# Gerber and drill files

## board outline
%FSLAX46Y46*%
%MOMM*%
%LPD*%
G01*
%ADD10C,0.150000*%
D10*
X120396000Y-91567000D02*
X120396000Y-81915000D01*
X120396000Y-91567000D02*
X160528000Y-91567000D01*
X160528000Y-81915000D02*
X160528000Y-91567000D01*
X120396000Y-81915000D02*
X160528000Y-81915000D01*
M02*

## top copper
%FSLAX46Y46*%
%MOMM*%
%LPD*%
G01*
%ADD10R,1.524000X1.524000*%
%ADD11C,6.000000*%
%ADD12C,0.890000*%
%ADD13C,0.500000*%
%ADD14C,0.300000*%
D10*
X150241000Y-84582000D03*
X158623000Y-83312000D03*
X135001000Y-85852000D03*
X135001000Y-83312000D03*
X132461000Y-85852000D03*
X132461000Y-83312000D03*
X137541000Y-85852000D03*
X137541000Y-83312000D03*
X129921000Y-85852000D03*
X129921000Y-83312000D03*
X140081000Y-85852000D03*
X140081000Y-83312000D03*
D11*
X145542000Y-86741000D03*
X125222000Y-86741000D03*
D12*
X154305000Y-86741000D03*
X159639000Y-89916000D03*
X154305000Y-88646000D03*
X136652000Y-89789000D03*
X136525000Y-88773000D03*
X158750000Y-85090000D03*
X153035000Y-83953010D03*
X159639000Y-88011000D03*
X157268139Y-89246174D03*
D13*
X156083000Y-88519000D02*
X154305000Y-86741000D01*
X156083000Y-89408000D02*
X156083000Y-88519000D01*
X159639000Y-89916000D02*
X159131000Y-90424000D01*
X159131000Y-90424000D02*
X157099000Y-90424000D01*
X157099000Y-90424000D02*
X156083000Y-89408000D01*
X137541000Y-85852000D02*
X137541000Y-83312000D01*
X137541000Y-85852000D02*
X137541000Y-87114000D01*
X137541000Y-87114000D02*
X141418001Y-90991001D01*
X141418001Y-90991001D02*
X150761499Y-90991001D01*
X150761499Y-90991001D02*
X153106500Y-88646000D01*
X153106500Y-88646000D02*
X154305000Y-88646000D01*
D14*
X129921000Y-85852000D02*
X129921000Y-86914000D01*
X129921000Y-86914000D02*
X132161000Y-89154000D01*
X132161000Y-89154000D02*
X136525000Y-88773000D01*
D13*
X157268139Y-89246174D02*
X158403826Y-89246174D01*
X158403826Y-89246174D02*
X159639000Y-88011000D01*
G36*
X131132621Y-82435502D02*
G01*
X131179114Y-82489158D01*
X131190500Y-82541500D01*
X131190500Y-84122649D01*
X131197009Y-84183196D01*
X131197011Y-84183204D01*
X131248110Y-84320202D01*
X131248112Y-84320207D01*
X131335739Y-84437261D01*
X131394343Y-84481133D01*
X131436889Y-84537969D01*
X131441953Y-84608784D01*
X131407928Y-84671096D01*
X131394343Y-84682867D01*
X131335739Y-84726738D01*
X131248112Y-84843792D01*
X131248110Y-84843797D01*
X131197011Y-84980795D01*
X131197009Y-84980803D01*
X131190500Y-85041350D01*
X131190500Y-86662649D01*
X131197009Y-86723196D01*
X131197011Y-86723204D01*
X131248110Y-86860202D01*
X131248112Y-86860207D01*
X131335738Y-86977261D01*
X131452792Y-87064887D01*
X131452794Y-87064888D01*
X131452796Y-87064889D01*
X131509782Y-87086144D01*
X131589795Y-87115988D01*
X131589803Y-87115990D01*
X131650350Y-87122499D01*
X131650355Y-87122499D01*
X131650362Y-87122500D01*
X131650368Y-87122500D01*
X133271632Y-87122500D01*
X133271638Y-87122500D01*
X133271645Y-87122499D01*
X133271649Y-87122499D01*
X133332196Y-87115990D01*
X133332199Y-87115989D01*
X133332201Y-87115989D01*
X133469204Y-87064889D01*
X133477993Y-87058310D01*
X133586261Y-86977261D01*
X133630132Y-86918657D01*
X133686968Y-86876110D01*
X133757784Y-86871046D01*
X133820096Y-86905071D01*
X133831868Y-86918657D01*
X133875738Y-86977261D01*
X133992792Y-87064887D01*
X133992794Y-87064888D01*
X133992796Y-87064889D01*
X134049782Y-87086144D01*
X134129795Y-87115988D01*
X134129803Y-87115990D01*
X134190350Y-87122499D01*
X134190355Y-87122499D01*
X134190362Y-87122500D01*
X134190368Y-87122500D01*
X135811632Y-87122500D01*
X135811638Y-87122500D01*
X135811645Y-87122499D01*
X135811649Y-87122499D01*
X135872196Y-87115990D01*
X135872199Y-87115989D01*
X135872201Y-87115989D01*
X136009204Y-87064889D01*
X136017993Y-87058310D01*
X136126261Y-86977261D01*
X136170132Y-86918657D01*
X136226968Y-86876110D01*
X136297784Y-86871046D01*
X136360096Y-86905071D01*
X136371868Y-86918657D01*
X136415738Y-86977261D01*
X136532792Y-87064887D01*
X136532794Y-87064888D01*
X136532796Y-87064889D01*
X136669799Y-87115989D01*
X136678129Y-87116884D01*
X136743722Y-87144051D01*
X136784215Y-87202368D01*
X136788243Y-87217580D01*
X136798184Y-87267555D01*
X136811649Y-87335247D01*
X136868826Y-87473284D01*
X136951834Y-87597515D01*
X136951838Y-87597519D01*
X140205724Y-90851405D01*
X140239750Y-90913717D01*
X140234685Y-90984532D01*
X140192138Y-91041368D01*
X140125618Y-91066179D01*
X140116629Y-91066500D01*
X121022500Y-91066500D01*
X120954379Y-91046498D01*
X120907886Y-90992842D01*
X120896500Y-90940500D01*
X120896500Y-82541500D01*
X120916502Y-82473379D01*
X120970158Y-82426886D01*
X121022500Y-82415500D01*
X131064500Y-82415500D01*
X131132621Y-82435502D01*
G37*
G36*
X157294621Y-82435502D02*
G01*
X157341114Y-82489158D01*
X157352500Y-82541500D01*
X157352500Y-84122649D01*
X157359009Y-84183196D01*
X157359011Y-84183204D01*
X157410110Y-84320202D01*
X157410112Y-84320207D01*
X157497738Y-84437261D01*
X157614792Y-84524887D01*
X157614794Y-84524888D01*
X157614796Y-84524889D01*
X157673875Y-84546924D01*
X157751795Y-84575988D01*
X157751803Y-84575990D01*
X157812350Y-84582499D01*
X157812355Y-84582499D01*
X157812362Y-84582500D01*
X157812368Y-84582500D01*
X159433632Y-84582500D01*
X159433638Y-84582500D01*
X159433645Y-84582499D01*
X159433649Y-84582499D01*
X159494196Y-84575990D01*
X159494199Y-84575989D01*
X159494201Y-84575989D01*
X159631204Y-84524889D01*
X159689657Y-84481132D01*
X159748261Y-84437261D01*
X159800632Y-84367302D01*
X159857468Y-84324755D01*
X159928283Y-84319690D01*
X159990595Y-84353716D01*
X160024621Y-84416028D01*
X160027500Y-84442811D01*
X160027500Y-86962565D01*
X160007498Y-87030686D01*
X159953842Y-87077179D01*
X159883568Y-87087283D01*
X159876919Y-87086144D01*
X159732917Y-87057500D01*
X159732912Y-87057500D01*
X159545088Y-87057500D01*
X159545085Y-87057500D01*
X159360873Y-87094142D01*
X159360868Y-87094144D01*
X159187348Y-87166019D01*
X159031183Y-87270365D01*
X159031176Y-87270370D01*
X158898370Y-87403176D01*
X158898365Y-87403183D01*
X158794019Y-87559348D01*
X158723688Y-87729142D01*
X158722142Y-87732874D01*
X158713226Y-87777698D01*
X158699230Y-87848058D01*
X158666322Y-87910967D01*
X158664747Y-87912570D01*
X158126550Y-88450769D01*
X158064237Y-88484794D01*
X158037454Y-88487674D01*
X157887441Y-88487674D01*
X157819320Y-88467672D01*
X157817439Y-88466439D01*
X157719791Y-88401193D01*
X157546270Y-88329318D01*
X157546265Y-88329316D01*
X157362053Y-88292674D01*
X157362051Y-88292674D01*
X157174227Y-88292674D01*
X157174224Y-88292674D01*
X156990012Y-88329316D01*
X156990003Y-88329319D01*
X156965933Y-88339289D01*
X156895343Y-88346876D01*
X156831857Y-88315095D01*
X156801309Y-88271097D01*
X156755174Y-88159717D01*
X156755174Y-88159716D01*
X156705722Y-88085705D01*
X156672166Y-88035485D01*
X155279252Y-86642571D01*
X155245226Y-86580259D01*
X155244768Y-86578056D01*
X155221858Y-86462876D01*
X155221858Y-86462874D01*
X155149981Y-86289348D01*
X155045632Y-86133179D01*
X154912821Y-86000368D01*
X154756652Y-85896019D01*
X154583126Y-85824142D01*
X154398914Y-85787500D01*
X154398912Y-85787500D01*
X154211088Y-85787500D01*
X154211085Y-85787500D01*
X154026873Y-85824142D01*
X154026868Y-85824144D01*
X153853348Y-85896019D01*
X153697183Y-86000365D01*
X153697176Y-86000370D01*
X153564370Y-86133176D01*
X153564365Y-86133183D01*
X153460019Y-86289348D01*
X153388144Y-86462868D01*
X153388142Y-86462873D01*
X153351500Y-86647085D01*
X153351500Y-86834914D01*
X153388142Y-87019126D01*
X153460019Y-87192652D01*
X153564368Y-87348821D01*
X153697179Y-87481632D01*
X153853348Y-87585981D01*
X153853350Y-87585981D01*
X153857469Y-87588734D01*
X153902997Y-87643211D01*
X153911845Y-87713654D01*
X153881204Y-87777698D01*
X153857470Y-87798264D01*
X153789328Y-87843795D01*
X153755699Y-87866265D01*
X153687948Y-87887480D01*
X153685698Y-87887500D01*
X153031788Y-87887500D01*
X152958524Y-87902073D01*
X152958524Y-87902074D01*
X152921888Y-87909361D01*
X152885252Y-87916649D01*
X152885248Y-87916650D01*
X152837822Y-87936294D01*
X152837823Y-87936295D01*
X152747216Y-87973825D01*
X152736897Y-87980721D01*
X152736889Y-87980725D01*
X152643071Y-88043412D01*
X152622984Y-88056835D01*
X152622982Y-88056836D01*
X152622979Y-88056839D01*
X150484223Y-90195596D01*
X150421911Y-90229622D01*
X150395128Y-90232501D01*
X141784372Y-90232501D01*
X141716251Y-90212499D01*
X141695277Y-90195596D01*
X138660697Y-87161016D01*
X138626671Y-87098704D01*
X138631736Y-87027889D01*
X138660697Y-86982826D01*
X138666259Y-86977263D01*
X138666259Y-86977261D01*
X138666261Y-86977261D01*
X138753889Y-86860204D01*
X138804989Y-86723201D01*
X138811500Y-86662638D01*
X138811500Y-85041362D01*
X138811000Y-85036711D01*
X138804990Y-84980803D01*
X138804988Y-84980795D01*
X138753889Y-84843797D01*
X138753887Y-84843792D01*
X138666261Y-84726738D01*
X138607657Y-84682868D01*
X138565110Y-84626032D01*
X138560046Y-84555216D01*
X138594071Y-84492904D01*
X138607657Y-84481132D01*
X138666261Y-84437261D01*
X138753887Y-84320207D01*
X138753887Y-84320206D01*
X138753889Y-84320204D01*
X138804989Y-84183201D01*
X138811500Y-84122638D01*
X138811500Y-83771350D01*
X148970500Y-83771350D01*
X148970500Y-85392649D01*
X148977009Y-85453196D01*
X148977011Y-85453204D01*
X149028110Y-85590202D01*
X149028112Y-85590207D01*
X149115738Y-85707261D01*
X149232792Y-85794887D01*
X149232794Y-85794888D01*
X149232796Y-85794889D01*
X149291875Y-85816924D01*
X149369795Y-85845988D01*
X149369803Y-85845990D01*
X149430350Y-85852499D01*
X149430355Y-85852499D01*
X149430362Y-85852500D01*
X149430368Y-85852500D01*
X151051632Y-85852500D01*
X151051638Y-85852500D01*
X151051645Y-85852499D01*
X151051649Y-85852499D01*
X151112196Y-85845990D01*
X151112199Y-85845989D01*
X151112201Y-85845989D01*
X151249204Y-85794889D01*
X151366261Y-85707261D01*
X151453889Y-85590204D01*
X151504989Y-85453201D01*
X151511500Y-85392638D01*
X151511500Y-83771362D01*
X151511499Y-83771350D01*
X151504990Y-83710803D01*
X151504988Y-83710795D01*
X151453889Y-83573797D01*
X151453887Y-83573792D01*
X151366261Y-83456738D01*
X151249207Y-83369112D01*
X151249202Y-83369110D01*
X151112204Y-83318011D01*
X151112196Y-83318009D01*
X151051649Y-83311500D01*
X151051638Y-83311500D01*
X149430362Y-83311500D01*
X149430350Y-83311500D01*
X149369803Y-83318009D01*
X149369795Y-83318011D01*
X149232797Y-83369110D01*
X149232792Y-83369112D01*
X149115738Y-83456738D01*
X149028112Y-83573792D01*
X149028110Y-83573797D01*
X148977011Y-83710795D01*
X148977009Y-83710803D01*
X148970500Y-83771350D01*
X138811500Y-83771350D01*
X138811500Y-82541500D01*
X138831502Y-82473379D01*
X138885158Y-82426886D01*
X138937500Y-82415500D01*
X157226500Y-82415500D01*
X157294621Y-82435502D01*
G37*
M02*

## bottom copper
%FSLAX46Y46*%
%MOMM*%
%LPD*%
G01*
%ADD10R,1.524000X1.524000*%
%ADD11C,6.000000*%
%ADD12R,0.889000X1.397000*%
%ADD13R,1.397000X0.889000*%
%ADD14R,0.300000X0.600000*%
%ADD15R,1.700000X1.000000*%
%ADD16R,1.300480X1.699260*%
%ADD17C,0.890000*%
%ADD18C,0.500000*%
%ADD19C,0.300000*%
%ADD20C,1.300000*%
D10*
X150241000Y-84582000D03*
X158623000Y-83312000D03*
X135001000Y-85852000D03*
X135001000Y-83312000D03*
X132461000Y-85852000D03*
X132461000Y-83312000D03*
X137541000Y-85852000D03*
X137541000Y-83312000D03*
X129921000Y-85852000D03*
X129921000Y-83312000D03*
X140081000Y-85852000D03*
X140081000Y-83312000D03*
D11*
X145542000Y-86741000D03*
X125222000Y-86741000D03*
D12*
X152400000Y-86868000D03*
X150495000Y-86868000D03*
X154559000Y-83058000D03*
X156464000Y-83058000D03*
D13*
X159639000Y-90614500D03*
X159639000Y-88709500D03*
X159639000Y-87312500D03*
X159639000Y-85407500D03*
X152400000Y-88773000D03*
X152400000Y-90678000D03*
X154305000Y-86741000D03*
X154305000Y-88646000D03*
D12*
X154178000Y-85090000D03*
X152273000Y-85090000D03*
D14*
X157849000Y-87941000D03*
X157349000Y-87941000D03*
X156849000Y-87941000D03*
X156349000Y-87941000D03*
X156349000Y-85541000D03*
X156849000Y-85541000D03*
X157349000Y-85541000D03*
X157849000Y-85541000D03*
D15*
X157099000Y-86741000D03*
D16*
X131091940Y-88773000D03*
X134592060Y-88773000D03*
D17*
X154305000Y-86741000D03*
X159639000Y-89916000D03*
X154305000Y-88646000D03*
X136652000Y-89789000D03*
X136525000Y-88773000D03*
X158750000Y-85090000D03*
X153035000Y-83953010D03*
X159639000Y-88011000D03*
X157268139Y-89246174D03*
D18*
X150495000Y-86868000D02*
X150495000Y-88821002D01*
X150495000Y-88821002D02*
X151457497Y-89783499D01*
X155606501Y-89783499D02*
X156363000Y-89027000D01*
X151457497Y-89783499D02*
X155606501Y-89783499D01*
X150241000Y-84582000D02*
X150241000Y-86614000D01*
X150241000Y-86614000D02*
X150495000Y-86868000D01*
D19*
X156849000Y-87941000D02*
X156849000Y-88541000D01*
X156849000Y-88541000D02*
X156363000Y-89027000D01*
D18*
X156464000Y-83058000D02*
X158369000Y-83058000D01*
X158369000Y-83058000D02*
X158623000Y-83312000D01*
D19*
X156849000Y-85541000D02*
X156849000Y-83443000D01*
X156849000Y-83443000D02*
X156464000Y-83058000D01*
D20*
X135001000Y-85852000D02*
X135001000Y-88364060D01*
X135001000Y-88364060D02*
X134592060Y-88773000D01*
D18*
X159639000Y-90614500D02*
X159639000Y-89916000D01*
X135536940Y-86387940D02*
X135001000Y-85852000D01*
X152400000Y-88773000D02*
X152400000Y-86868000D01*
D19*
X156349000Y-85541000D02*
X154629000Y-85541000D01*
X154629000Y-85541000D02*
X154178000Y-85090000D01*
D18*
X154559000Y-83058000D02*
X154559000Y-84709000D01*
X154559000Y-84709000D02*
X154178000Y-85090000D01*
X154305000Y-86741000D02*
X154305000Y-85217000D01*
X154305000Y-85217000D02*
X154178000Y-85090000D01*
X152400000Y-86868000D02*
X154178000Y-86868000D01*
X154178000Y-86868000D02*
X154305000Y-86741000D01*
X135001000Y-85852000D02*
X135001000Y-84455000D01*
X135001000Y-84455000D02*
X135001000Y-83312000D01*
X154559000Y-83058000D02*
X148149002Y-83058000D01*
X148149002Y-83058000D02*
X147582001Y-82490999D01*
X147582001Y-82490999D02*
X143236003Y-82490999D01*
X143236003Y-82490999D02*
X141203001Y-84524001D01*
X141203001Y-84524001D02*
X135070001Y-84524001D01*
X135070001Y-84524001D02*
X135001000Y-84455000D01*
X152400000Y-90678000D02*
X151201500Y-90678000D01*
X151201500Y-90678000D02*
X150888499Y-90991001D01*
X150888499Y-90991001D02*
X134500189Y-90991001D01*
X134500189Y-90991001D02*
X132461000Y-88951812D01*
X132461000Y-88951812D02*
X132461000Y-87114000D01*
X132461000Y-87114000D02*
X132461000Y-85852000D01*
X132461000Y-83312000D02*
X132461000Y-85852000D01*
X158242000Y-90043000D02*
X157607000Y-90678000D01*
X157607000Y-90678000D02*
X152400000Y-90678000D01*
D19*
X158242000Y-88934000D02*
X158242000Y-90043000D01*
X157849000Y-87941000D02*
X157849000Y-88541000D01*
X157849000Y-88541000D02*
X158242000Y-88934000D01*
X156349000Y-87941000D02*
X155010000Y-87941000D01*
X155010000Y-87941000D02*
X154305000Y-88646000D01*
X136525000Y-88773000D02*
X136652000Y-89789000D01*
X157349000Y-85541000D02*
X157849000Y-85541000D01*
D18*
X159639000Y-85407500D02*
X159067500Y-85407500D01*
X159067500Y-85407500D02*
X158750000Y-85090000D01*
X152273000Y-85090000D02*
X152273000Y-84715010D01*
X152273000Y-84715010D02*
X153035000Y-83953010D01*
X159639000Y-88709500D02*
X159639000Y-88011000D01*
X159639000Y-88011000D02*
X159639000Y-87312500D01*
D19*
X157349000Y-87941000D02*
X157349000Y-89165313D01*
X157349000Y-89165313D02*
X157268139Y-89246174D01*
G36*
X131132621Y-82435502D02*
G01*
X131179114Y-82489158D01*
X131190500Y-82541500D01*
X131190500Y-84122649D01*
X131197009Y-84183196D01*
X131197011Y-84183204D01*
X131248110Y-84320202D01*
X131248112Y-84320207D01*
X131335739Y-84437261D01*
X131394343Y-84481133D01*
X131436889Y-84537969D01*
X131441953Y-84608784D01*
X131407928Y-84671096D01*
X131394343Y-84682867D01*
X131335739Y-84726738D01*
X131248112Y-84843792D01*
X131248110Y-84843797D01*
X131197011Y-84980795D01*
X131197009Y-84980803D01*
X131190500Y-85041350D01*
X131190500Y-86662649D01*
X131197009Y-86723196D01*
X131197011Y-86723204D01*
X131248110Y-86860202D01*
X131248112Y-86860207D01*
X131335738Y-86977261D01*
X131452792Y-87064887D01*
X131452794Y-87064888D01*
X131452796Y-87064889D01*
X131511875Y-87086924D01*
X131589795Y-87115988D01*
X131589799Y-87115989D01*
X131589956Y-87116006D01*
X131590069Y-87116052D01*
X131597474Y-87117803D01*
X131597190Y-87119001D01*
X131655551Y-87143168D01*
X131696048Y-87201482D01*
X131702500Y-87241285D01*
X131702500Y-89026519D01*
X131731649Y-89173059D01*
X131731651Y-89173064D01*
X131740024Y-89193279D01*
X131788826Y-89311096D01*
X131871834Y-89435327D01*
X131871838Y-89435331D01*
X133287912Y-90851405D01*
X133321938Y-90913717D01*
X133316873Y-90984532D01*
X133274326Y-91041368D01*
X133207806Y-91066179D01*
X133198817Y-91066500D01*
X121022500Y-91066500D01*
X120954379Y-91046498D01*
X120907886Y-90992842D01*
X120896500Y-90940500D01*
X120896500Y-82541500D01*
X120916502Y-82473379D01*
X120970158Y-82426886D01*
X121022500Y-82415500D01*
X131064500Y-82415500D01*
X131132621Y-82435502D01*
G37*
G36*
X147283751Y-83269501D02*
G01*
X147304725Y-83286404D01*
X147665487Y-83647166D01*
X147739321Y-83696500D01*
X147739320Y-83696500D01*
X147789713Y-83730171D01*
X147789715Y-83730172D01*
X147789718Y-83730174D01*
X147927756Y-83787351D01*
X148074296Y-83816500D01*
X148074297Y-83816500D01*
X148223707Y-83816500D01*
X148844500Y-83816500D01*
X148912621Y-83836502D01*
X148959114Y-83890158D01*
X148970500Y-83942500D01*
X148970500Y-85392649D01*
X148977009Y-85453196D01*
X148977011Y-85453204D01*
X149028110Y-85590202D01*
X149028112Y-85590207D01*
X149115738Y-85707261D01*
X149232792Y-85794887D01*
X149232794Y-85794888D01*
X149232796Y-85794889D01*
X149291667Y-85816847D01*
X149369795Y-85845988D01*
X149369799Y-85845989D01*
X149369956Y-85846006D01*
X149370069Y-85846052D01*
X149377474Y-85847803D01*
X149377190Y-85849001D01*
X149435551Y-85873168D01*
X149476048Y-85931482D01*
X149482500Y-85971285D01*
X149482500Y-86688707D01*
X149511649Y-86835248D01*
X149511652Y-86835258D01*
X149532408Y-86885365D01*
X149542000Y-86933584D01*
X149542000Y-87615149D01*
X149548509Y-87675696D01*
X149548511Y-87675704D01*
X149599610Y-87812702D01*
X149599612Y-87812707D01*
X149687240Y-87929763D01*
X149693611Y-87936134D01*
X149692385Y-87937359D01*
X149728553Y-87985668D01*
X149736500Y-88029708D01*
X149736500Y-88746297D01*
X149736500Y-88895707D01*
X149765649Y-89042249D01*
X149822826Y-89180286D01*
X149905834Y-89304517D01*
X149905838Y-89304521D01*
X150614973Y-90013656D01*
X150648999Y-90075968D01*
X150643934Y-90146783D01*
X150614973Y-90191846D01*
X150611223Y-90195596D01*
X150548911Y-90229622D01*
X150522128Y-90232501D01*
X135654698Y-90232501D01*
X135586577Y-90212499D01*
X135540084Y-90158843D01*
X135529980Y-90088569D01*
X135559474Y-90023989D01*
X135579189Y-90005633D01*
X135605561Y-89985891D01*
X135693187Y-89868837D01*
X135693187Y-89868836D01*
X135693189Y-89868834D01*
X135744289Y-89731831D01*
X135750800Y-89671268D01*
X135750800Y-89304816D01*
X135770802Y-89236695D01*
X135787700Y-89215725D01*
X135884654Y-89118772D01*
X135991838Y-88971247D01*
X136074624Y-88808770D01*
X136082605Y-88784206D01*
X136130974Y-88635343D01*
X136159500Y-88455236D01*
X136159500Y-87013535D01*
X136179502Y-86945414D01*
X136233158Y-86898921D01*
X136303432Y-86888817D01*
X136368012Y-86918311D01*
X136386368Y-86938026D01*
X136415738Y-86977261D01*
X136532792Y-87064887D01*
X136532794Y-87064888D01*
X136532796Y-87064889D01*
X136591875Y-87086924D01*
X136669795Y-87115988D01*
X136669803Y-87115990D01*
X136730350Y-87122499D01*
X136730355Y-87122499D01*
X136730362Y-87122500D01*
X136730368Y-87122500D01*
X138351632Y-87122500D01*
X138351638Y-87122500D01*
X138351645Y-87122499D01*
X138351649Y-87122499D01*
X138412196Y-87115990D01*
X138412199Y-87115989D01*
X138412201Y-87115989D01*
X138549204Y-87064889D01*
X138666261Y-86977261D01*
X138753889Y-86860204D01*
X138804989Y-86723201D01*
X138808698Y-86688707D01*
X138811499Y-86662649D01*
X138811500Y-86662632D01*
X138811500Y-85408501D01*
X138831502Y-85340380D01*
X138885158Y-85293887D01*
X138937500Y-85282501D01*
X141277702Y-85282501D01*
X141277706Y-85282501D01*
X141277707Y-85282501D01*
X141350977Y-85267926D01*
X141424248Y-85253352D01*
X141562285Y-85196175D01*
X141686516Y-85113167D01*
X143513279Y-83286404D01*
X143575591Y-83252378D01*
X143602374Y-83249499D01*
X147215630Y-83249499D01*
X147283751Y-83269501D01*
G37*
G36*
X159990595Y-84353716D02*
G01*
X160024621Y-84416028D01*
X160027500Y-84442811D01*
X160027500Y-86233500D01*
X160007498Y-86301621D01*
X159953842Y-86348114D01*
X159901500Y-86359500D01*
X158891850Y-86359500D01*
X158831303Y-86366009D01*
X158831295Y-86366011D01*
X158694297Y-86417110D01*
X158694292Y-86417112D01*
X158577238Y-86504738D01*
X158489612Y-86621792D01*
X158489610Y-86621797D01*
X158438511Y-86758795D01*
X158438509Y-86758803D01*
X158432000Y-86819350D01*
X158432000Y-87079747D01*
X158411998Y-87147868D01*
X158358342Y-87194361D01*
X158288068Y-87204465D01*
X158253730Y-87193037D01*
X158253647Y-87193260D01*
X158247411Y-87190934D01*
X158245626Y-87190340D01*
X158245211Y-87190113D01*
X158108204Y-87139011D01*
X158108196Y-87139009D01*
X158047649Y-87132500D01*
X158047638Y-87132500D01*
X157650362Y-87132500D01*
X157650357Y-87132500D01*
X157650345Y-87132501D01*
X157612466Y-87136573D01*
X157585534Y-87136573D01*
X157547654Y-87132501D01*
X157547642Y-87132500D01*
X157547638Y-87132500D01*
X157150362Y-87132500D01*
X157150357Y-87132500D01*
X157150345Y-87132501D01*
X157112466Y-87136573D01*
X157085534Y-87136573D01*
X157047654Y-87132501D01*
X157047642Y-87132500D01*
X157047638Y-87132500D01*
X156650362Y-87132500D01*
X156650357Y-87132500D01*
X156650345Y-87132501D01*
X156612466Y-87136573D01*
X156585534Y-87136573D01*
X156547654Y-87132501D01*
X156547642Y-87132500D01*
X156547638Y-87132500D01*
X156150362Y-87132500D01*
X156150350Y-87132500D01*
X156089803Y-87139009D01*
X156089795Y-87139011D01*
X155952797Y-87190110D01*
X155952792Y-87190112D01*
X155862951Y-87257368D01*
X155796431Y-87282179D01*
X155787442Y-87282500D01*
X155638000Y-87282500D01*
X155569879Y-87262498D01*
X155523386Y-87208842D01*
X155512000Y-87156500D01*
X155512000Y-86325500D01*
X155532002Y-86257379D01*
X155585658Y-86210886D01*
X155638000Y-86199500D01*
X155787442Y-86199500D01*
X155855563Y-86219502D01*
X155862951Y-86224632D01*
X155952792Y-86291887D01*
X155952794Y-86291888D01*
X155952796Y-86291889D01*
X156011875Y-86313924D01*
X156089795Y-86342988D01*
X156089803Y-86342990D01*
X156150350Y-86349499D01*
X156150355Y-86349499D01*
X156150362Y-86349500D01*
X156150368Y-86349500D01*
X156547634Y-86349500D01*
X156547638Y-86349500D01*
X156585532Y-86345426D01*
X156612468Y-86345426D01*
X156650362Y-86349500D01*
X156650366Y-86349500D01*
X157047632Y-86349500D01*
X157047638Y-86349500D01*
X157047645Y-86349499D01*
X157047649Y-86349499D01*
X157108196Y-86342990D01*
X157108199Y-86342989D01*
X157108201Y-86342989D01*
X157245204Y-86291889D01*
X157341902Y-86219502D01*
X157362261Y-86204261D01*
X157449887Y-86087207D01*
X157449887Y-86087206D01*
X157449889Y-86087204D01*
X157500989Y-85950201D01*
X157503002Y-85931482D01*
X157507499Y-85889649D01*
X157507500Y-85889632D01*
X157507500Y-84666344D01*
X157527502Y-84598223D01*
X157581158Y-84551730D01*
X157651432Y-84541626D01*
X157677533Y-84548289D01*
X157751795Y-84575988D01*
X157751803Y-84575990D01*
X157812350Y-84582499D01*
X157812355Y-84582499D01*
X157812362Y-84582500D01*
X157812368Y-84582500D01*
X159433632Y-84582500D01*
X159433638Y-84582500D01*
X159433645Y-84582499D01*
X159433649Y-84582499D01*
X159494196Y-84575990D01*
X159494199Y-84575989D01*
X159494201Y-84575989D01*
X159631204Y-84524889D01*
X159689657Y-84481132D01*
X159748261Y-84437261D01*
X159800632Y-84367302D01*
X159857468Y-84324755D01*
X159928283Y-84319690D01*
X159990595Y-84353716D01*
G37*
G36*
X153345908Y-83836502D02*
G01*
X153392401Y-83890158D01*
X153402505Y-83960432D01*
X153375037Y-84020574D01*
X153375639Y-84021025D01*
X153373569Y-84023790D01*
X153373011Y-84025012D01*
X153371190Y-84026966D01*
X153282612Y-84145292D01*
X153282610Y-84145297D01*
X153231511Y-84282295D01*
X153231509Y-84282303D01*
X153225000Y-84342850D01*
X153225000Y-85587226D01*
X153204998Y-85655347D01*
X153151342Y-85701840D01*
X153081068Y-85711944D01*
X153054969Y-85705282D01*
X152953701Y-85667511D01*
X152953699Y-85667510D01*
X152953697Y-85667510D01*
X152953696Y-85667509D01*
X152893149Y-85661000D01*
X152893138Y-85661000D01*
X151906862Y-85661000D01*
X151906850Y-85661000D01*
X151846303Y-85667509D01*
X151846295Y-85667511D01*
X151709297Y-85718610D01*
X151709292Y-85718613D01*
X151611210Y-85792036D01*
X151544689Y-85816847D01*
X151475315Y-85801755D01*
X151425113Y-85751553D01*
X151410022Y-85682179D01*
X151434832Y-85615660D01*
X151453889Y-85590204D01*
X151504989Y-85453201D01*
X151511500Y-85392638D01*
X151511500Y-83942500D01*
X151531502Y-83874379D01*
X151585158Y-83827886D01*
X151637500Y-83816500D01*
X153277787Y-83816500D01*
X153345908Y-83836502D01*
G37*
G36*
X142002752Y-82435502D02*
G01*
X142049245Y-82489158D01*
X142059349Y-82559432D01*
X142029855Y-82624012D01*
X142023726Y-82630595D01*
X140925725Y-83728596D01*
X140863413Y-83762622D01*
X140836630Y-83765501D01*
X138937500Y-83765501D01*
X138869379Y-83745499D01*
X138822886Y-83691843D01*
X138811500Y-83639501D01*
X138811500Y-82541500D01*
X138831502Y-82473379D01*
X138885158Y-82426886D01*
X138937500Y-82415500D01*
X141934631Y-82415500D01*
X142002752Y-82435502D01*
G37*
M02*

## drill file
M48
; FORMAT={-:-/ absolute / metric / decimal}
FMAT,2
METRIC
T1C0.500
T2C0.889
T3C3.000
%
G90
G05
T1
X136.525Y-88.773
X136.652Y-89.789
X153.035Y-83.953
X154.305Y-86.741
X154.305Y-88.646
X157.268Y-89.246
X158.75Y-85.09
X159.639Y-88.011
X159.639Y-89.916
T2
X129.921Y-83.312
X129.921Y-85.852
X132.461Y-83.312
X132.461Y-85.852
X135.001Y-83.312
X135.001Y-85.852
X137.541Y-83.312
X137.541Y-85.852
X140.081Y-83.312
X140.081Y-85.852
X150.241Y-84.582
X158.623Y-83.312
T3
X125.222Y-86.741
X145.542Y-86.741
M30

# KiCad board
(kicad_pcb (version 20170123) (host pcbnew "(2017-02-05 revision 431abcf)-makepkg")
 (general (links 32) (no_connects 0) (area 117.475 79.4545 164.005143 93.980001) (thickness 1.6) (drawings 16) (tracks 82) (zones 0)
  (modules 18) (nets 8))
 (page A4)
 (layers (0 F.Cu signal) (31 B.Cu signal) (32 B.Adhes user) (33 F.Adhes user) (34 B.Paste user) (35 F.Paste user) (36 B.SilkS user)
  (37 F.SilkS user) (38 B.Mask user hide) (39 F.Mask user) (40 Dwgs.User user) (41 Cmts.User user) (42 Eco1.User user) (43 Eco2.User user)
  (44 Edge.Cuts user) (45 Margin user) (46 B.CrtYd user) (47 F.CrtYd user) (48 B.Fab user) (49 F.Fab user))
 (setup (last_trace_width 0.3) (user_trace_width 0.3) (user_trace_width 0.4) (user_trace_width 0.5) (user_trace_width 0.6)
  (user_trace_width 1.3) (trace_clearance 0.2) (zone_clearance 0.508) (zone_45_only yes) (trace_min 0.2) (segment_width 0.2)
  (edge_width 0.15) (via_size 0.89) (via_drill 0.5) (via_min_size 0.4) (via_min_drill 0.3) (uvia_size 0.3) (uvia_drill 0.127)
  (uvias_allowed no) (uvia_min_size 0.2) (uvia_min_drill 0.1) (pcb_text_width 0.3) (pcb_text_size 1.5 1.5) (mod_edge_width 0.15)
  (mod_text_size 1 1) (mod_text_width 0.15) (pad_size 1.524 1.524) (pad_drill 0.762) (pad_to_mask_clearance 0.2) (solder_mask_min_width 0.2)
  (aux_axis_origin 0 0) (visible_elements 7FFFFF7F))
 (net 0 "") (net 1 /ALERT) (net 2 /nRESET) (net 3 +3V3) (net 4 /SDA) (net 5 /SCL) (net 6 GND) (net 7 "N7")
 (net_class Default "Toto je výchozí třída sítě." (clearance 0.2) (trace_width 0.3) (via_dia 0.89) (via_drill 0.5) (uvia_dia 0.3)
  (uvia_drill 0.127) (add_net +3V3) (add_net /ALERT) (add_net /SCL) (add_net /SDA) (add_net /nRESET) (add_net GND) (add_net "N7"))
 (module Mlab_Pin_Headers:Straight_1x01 (layer F.Cu) (at 150.241 84.582)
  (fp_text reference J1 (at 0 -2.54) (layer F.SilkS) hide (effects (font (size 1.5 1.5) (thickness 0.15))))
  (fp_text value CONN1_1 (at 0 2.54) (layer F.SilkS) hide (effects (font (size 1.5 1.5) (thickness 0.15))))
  (pad 1 thru_hole rect (at 0 0) (size 1.524 1.524) (drill 0.889) (layers *.Cu *.Mask F.SilkS) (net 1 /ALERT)))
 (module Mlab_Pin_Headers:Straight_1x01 (layer F.Cu) (at 158.623 83.312)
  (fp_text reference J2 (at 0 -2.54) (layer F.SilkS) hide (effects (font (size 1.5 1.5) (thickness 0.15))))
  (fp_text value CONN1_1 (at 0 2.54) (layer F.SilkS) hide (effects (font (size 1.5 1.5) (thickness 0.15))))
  (pad 1 thru_hole rect (at 0 0) (size 1.524 1.524) (drill 0.889) (layers *.Cu *.Mask F.SilkS) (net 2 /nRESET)))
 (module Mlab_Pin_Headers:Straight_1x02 (layer F.Cu) (at 135.001 84.582)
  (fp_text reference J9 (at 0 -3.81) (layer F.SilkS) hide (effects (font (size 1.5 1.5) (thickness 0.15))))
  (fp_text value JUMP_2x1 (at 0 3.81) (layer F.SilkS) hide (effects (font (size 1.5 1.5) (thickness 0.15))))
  (pad 2 thru_hole rect (at 0 1.27) (size 1.524 1.524) (drill 0.889) (layers *.Cu *.Mask F.SilkS) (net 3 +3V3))
  (pad 1 thru_hole rect (at 0 -1.27) (size 1.524 1.524) (drill 0.889) (layers *.Cu *.Mask F.SilkS) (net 3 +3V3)))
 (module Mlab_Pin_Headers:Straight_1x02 (layer F.Cu) (at 132.461 84.582)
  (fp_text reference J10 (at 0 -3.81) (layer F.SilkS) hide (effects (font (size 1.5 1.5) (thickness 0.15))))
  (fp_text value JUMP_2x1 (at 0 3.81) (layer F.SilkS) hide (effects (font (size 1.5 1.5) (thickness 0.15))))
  (pad 2 thru_hole rect (at 0 1.27) (size 1.524 1.524) (drill 0.889) (layers *.Cu *.Mask F.SilkS) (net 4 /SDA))
  (pad 1 thru_hole rect (at 0 -1.27) (size 1.524 1.524) (drill 0.889) (layers *.Cu *.Mask F.SilkS) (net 4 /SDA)))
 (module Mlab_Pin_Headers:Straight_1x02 (layer F.Cu) (at 137.541 84.582)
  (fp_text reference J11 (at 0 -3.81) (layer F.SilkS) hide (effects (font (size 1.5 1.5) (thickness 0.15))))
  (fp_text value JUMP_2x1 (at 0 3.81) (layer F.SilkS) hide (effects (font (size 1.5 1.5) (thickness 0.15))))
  (pad 2 thru_hole rect (at 0 1.27) (size 1.524 1.524) (drill 0.889) (layers *.Cu *.Mask F.SilkS) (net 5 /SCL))
  (pad 1 thru_hole rect (at 0 -1.27) (size 1.524 1.524) (drill 0.889) (layers *.Cu *.Mask F.SilkS) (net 5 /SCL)))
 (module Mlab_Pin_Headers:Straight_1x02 (layer F.Cu) (at 129.921 84.582)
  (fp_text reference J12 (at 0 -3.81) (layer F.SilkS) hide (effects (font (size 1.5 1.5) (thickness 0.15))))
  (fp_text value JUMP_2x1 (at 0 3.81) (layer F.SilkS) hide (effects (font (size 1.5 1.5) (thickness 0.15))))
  (pad 2 thru_hole rect (at 0 1.27) (size 1.524 1.524) (drill 0.889) (layers *.Cu *.Mask F.SilkS) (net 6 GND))
  (pad 1 thru_hole rect (at 0 -1.27) (size 1.524 1.524) (drill 0.889) (layers *.Cu *.Mask F.SilkS) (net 6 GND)))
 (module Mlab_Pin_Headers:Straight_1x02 (layer F.Cu) (at 140.081 84.582)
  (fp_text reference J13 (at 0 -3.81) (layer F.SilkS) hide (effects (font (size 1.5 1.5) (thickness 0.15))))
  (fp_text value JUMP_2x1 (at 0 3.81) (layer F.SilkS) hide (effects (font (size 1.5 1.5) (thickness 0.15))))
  (pad 2 thru_hole rect (at 0 1.27) (size 1.524 1.524) (drill 0.889) (layers *.Cu *.Mask F.SilkS) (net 6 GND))
  (pad 1 thru_hole rect (at 0 -1.27) (size 1.524 1.524) (drill 0.889) (layers *.Cu *.Mask F.SilkS) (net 6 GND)))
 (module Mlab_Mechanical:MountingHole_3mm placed (layer F.Cu) (at 145.542 86.741)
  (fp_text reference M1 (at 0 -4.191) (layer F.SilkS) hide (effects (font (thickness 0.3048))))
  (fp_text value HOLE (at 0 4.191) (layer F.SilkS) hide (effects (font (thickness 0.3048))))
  (pad 1 thru_hole circle (at 0 0) (size 6 6) (drill 3) (layers *.Cu *.Adhes *.Mask) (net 6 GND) (clearance 1) (zone_connect 2)))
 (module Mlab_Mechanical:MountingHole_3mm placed (layer F.Cu) (at 125.222 86.741)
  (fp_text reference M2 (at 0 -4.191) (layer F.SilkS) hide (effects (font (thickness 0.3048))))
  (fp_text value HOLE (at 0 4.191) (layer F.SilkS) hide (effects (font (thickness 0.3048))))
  (pad 1 thru_hole circle (at 0 0) (size 6 6) (drill 3) (layers *.Cu *.Adhes *.Mask) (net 6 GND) (clearance 1) (zone_connect 2)))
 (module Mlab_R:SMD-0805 (layer B.Cu) (at 151.4475 86.868 180)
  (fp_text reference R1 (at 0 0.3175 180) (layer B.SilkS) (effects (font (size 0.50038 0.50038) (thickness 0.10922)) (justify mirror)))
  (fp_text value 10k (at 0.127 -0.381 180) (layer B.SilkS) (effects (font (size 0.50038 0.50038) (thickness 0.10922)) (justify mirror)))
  (pad 1 smd rect (at -0.9525 0 180) (size 0.889 1.397) (layers B.Cu B.Paste B.Mask) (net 3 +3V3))
  (pad 2 smd rect (at 0.9525 0 180) (size 0.889 1.397) (layers B.Cu B.Paste B.Mask) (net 1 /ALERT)))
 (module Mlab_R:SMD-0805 (layer B.Cu) (at 155.5115 83.058)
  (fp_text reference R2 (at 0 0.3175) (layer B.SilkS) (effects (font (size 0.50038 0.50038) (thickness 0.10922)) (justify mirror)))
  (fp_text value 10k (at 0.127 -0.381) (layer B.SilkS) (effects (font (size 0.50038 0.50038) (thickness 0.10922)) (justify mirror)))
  (pad 1 smd rect (at -0.9525 0) (size 0.889 1.397) (layers B.Cu B.Paste B.Mask) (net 3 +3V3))
  (pad 2 smd rect (at 0.9525 0) (size 0.889 1.397) (layers B.Cu B.Paste B.Mask) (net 2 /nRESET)))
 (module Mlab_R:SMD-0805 (layer B.Cu) (at 159.639 89.662 90)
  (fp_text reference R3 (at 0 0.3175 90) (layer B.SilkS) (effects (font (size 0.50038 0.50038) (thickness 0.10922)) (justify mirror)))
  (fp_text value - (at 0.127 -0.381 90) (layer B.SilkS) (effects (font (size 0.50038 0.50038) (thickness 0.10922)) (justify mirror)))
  (pad 1 smd rect (at -0.9525 0 90) (size 0.889 1.397) (layers B.Cu B.Paste B.Mask) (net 3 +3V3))
  (pad 2 smd rect (at 0.9525 0 90) (size 0.889 1.397) (layers B.Cu B.Paste B.Mask) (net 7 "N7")))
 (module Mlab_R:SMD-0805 (layer B.Cu) (at 159.639 86.36 90)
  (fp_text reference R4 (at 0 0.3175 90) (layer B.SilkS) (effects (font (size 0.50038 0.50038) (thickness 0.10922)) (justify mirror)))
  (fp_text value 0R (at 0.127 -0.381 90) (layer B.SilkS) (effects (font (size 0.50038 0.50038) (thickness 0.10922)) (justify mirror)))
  (pad 1 smd rect (at -0.9525 0 90) (size 0.889 1.397) (layers B.Cu B.Paste B.Mask) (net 7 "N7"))
  (pad 2 smd rect (at 0.9525 0 90) (size 0.889 1.397) (layers B.Cu B.Paste B.Mask) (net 6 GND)))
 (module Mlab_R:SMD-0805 (layer B.Cu) (at 152.4 89.7255 270)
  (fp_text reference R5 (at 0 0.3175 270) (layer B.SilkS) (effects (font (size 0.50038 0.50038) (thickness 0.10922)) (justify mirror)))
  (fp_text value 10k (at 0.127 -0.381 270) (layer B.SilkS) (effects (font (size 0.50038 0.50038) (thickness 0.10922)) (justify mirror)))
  (pad 1 smd rect (at -0.9525 0 270) (size 0.889 1.397) (layers B.Cu B.Paste B.Mask) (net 3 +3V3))
  (pad 2 smd rect (at 0.9525 0 270) (size 0.889 1.397) (layers B.Cu B.Paste B.Mask) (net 4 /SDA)))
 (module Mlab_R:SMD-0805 (layer B.Cu) (at 154.305 87.6935 270)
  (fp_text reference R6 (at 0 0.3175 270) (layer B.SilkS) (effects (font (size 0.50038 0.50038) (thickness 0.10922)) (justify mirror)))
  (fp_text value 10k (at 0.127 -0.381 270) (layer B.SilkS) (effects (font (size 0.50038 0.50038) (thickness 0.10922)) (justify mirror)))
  (pad 1 smd rect (at -0.9525 0 270) (size 0.889 1.397) (layers B.Cu B.Paste B.Mask) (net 3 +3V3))
  (pad 2 smd rect (at 0.9525 0 270) (size 0.889 1.397) (layers B.Cu B.Paste B.Mask) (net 5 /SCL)))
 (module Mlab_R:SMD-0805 (layer B.Cu) (at 153.2255 85.09 180)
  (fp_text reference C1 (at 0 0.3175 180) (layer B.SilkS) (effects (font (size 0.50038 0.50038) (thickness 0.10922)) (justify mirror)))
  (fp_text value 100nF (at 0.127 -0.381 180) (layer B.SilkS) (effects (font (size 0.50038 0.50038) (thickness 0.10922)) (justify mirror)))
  (pad 1 smd rect (at -0.9525 0 180) (size 0.889 1.397) (layers B.Cu B.Paste B.Mask) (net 3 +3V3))
  (pad 2 smd rect (at 0.9525 0 180) (size 0.889 1.397) (layers B.Cu B.Paste B.Mask) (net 6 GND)))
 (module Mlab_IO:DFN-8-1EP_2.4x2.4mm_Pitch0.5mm (layer B.Cu) (at 157.099 86.741 90)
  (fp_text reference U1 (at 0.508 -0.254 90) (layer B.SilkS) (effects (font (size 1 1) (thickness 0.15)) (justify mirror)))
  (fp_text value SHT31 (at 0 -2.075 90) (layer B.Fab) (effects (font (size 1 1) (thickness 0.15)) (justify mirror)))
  (pad 1 smd rect (at -1.2 0.75 90) (size 0.6 0.3) (layers B.Cu B.Paste B.Mask) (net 4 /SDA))
  (pad 2 smd rect (at -1.2 0.25 90) (size 0.6 0.3) (layers B.Cu B.Paste B.Mask) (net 7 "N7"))
  (pad 3 smd rect (at -1.2 -0.25 90) (size 0.6 0.3) (layers B.Cu B.Paste B.Mask) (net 1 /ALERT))
  (pad 4 smd rect (at -1.2 -0.75 90) (size 0.6 0.3) (layers B.Cu B.Paste B.Mask) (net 5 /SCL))
  (pad 5 smd rect (at 1.2 -0.75 90) (size 0.6 0.3) (layers B.Cu B.Paste B.Mask) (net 3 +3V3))
  (pad 6 smd rect (at 1.2 -0.25 90) (size 0.6 0.3) (layers B.Cu B.Paste B.Mask) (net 2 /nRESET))
  (pad 7 smd rect (at 1.2 0.25 90) (size 0.6 0.3) (layers B.Cu B.Paste B.Mask) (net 6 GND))
  (pad 8 smd rect (at 1.2 0.75 90) (size 0.6 0.3) (layers B.Cu B.Paste B.Mask) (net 6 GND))
  (pad 9 smd rect (at 0 0 90) (size 1 1.7) (layers B.Cu B.Paste B.Mask) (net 6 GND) (solder_paste_margin_ratio -0.2)))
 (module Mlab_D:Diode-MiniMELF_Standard (layer B.Cu) (at 132.842 88.773)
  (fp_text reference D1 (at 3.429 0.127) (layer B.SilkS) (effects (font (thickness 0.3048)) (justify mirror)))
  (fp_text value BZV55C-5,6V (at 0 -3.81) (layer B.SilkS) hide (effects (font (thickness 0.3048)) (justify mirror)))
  (pad 1 smd rect (at -1.75006 0) (size 1.30048 1.69926) (layers B.Cu B.Paste B.Mask) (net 6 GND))
  (pad 2 smd rect (at 1.75006 0) (size 1.30048 1.69926) (layers B.Cu B.Paste B.Mask) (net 3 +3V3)))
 (gr_line (start 120.396 91.567) (end 120.396 81.915) (angle 90) (layer Edge.Cuts) (width 0.15))
 (gr_line (start 120.396 91.567) (end 160.528 91.567) (angle 90) (layer Edge.Cuts) (width 0.15))
 (gr_line (start 160.528 81.915) (end 160.528 91.567) (angle 90) (layer Edge.Cuts) (width 0.15))
 (gr_line (start 120.396 81.915) (end 160.528 81.915) (angle 90) (layer Edge.Cuts) (width 0.15))
 (segment (start 150.495 86.868) (end 150.495 88.821002) (width 0.5) (layer B.Cu) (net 1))
 (segment (start 150.495 88.821002) (end 151.457497 89.783499) (width 0.5) (layer B.Cu) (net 1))
 (segment (start 155.606501 89.783499) (end 156.363 89.027) (width 0.5) (layer B.Cu) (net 1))
 (segment (start 151.457497 89.783499) (end 155.606501 89.783499) (width 0.5) (layer B.Cu) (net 1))
 (segment (start 150.241 84.582) (end 150.241 86.614) (width 0.5) (layer B.Cu) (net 1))
 (segment (start 150.241 86.614) (end 150.495 86.868) (width 0.5) (layer B.Cu) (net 1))
 (segment (start 156.849 87.941) (end 156.849 88.541) (width 0.3) (layer B.Cu) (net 1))
 (segment (start 156.849 88.541) (end 156.363 89.027) (width 0.3) (layer B.Cu) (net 1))
 (segment (start 156.464 83.058) (end 158.369 83.058) (width 0.5) (layer B.Cu) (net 2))
 (segment (start 158.369 83.058) (end 158.623 83.312) (width 0.5) (layer B.Cu) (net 2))
 (segment (start 156.849 85.541) (end 156.849 83.443) (width 0.3) (layer B.Cu) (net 2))
 (segment (start 156.849 83.443) (end 156.464 83.058) (width 0.3) (layer B.Cu) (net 2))
 (segment (start 135.001 85.852) (end 135.001 88.36406) (width 1.3) (layer B.Cu) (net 3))
 (segment (start 135.001 88.36406) (end 134.59206 88.773) (width 1.3) (layer B.Cu) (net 3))
 (segment (start 156.083 88.519) (end 154.305 86.741) (width 0.5) (layer F.Cu) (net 3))
 (segment (start 156.083 89.408) (end 156.083 88.519) (width 0.5) (layer F.Cu) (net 3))
 (segment (start 159.639 89.916) (end 159.131 90.424) (width 0.5) (layer F.Cu) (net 3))
 (segment (start 159.131 90.424) (end 157.099 90.424) (width 0.5) (layer F.Cu) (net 3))
 (segment (start 157.099 90.424) (end 156.083 89.408) (width 0.5) (layer F.Cu) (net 3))
 (via (at 154.305 86.741) (size 0.89) (drill 0.5) (layers F.Cu B.Cu) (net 3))
 (segment (start 159.639 90.6145) (end 159.639 89.916) (width 0.5) (layer B.Cu) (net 3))
 (via (at 159.639 89.916) (size 0.89) (drill 0.5) (layers F.Cu B.Cu) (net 3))
 (segment (start 135.53694 86.38794) (end 135.001 85.852) (width 0.5) (layer B.Cu) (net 3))
 (segment (start 152.4 88.773) (end 152.4 86.868) (width 0.5) (layer B.Cu) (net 3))
 (segment (start 156.349 85.541) (end 154.629 85.541) (width 0.3) (layer B.Cu) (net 3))
 (segment (start 154.629 85.541) (end 154.178 85.09) (width 0.3) (layer B.Cu) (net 3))
 (segment (start 154.559 83.058) (end 154.559 84.709) (width 0.5) (layer B.Cu) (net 3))
 (segment (start 154.559 84.709) (end 154.178 85.09) (width 0.5) (layer B.Cu) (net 3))
 (segment (start 154.305 86.741) (end 154.305 85.217) (width 0.5) (layer B.Cu) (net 3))
 (segment (start 154.305 85.217) (end 154.178 85.09) (width 0.5) (layer B.Cu) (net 3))
 (segment (start 152.4 86.868) (end 154.178 86.868) (width 0.5) (layer B.Cu) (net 3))
 (segment (start 154.178 86.868) (end 154.305 86.741) (width 0.5) (layer B.Cu) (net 3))
 (segment (start 135.001 85.852) (end 135.001 84.455) (width 0.5) (layer B.Cu) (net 3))
 (segment (start 135.001 84.455) (end 135.001 83.312) (width 0.5) (layer B.Cu) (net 3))
 (segment (start 154.559 83.058) (end 148.149002 83.058) (width 0.5) (layer B.Cu) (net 3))
 (segment (start 148.149002 83.058) (end 147.582001 82.490999) (width 0.5) (layer B.Cu) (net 3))
 (segment (start 147.582001 82.490999) (end 143.236003 82.490999) (width 0.5) (layer B.Cu) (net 3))
 (segment (start 143.236003 82.490999) (end 141.203001 84.524001) (width 0.5) (layer B.Cu) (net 3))
 (segment (start 141.203001 84.524001) (end 135.070001 84.524001) (width 0.5) (layer B.Cu) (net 3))
 (segment (start 135.070001 84.524001) (end 135.001 84.455) (width 0.5) (layer B.Cu) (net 3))
 (segment (start 152.4 90.678) (end 151.2015 90.678) (width 0.5) (layer B.Cu) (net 4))
 (segment (start 151.2015 90.678) (end 150.888499 90.991001) (width 0.5) (layer B.Cu) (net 4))
 (segment (start 150.888499 90.991001) (end 134.500189 90.991001) (width 0.5) (layer B.Cu) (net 4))
 (segment (start 134.500189 90.991001) (end 132.461 88.951812) (width 0.5) (layer B.Cu) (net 4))
 (segment (start 132.461 88.951812) (end 132.461 87.114) (width 0.5) (layer B.Cu) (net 4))
 (segment (start 132.461 87.114) (end 132.461 85.852) (width 0.5) (layer B.Cu) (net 4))
 (segment (start 132.461 83.312) (end 132.461 85.852) (width 0.5) (layer B.Cu) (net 4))
 (segment (start 158.242 90.043) (end 157.607 90.678) (width 0.5) (layer B.Cu) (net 4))
 (segment (start 157.607 90.678) (end 152.4 90.678) (width 0.5) (layer B.Cu) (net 4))
 (segment (start 158.242 88.934) (end 158.242 90.043) (width 0.3) (layer B.Cu) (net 4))
 (segment (start 157.849 87.941) (end 157.849 88.541) (width 0.3) (layer B.Cu) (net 4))
 (segment (start 157.849 88.541) (end 158.242 88.934) (width 0.3) (layer B.Cu) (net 4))
 (segment (start 137.541 85.852) (end 137.541 83.312) (width 0.5) (layer F.Cu) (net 5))
 (segment (start 137.541 85.852) (end 137.541 87.114) (width 0.5) (layer F.Cu) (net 5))
 (segment (start 137.541 87.114) (end 141.418001 90.991001) (width 0.5) (layer F.Cu) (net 5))
 (segment (start 141.418001 90.991001) (end 150.761499 90.991001) (width 0.5) (layer F.Cu) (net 5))
 (segment (start 150.761499 90.991001) (end 153.1065 88.646) (width 0.5) (layer F.Cu) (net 5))
 (segment (start 153.1065 88.646) (end 154.305 88.646) (width 0.5) (layer F.Cu) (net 5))
 (via (at 154.305 88.646) (size 0.89) (drill 0.5) (layers F.Cu B.Cu) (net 5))
 (segment (start 156.349 87.941) (end 155.01 87.941) (width 0.3) (layer B.Cu) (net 5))
 (segment (start 155.01 87.941) (end 154.305 88.646) (width 0.3) (layer B.Cu) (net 5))
 (segment (start 136.525 88.773) (end 136.652 89.789) (width 0.3) (layer B.Cu) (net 6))
 (via (at 136.652 89.789) (size 0.89) (drill 0.5) (layers F.Cu B.Cu) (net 6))
 (segment (start 129.921 85.852) (end 129.921 86.914) (width 0.3) (layer F.Cu) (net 6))
 (segment (start 129.921 86.914) (end 132.161 89.154) (width 0.3) (layer F.Cu) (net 6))
 (segment (start 132.161 89.154) (end 136.525 88.773) (width 0.3) (layer F.Cu) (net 6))
 (via (at 136.525 88.773) (size 0.89) (drill 0.5) (layers F.Cu B.Cu) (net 6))
 (segment (start 157.349 85.541) (end 157.849 85.541) (width 0.3) (layer B.Cu) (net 6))
 (segment (start 159.639 85.4075) (end 159.0675 85.4075) (width 0.5) (layer B.Cu) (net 6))
 (segment (start 159.0675 85.4075) (end 158.75 85.09) (width 0.5) (layer B.Cu) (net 6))
 (via (at 158.75 85.09) (size 0.89) (drill 0.5) (layers F.Cu B.Cu) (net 6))
 (segment (start 152.273 85.09) (end 152.273 84.71501) (width 0.5) (layer B.Cu) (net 6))
 (segment (start 152.273 84.71501) (end 153.035 83.95301) (width 0.5) (layer B.Cu) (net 6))
 (via (at 153.035 83.95301) (size 0.89) (drill 0.5) (layers F.Cu B.Cu) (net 6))
 (segment (start 159.639 88.7095) (end 159.639 88.011) (width 0.5) (layer B.Cu) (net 7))
 (segment (start 159.639 88.011) (end 159.639 87.3125) (width 0.5) (layer B.Cu) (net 7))
 (segment (start 157.268139 89.246174) (end 158.403826 89.246174) (width 0.5) (layer F.Cu) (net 7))
 (segment (start 158.403826 89.246174) (end 159.639 88.011) (width 0.5) (layer F.Cu) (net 7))
 (via (at 159.639 88.011) (size 0.89) (drill 0.5) (layers F.Cu B.Cu) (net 7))
 (segment (start 157.349 87.941) (end 157.349 89.165313) (width 0.3) (layer B.Cu) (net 7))
 (segment (start 157.349 89.165313) (end 157.268139 89.246174) (width 0.3) (layer B.Cu) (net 7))
 (via (at 157.268139 89.246174) (size 0.89) (drill 0.5) (layers F.Cu B.Cu) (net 7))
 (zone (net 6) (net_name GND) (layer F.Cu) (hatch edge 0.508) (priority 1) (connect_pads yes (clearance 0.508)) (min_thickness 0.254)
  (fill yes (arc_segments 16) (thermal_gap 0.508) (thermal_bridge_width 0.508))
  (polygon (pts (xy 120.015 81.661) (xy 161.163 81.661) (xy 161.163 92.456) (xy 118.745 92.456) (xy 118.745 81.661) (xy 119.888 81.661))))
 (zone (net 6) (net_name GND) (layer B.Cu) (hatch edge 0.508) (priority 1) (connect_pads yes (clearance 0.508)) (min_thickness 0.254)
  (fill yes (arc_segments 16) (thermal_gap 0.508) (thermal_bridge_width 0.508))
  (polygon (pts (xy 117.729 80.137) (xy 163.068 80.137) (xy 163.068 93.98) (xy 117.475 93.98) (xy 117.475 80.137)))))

